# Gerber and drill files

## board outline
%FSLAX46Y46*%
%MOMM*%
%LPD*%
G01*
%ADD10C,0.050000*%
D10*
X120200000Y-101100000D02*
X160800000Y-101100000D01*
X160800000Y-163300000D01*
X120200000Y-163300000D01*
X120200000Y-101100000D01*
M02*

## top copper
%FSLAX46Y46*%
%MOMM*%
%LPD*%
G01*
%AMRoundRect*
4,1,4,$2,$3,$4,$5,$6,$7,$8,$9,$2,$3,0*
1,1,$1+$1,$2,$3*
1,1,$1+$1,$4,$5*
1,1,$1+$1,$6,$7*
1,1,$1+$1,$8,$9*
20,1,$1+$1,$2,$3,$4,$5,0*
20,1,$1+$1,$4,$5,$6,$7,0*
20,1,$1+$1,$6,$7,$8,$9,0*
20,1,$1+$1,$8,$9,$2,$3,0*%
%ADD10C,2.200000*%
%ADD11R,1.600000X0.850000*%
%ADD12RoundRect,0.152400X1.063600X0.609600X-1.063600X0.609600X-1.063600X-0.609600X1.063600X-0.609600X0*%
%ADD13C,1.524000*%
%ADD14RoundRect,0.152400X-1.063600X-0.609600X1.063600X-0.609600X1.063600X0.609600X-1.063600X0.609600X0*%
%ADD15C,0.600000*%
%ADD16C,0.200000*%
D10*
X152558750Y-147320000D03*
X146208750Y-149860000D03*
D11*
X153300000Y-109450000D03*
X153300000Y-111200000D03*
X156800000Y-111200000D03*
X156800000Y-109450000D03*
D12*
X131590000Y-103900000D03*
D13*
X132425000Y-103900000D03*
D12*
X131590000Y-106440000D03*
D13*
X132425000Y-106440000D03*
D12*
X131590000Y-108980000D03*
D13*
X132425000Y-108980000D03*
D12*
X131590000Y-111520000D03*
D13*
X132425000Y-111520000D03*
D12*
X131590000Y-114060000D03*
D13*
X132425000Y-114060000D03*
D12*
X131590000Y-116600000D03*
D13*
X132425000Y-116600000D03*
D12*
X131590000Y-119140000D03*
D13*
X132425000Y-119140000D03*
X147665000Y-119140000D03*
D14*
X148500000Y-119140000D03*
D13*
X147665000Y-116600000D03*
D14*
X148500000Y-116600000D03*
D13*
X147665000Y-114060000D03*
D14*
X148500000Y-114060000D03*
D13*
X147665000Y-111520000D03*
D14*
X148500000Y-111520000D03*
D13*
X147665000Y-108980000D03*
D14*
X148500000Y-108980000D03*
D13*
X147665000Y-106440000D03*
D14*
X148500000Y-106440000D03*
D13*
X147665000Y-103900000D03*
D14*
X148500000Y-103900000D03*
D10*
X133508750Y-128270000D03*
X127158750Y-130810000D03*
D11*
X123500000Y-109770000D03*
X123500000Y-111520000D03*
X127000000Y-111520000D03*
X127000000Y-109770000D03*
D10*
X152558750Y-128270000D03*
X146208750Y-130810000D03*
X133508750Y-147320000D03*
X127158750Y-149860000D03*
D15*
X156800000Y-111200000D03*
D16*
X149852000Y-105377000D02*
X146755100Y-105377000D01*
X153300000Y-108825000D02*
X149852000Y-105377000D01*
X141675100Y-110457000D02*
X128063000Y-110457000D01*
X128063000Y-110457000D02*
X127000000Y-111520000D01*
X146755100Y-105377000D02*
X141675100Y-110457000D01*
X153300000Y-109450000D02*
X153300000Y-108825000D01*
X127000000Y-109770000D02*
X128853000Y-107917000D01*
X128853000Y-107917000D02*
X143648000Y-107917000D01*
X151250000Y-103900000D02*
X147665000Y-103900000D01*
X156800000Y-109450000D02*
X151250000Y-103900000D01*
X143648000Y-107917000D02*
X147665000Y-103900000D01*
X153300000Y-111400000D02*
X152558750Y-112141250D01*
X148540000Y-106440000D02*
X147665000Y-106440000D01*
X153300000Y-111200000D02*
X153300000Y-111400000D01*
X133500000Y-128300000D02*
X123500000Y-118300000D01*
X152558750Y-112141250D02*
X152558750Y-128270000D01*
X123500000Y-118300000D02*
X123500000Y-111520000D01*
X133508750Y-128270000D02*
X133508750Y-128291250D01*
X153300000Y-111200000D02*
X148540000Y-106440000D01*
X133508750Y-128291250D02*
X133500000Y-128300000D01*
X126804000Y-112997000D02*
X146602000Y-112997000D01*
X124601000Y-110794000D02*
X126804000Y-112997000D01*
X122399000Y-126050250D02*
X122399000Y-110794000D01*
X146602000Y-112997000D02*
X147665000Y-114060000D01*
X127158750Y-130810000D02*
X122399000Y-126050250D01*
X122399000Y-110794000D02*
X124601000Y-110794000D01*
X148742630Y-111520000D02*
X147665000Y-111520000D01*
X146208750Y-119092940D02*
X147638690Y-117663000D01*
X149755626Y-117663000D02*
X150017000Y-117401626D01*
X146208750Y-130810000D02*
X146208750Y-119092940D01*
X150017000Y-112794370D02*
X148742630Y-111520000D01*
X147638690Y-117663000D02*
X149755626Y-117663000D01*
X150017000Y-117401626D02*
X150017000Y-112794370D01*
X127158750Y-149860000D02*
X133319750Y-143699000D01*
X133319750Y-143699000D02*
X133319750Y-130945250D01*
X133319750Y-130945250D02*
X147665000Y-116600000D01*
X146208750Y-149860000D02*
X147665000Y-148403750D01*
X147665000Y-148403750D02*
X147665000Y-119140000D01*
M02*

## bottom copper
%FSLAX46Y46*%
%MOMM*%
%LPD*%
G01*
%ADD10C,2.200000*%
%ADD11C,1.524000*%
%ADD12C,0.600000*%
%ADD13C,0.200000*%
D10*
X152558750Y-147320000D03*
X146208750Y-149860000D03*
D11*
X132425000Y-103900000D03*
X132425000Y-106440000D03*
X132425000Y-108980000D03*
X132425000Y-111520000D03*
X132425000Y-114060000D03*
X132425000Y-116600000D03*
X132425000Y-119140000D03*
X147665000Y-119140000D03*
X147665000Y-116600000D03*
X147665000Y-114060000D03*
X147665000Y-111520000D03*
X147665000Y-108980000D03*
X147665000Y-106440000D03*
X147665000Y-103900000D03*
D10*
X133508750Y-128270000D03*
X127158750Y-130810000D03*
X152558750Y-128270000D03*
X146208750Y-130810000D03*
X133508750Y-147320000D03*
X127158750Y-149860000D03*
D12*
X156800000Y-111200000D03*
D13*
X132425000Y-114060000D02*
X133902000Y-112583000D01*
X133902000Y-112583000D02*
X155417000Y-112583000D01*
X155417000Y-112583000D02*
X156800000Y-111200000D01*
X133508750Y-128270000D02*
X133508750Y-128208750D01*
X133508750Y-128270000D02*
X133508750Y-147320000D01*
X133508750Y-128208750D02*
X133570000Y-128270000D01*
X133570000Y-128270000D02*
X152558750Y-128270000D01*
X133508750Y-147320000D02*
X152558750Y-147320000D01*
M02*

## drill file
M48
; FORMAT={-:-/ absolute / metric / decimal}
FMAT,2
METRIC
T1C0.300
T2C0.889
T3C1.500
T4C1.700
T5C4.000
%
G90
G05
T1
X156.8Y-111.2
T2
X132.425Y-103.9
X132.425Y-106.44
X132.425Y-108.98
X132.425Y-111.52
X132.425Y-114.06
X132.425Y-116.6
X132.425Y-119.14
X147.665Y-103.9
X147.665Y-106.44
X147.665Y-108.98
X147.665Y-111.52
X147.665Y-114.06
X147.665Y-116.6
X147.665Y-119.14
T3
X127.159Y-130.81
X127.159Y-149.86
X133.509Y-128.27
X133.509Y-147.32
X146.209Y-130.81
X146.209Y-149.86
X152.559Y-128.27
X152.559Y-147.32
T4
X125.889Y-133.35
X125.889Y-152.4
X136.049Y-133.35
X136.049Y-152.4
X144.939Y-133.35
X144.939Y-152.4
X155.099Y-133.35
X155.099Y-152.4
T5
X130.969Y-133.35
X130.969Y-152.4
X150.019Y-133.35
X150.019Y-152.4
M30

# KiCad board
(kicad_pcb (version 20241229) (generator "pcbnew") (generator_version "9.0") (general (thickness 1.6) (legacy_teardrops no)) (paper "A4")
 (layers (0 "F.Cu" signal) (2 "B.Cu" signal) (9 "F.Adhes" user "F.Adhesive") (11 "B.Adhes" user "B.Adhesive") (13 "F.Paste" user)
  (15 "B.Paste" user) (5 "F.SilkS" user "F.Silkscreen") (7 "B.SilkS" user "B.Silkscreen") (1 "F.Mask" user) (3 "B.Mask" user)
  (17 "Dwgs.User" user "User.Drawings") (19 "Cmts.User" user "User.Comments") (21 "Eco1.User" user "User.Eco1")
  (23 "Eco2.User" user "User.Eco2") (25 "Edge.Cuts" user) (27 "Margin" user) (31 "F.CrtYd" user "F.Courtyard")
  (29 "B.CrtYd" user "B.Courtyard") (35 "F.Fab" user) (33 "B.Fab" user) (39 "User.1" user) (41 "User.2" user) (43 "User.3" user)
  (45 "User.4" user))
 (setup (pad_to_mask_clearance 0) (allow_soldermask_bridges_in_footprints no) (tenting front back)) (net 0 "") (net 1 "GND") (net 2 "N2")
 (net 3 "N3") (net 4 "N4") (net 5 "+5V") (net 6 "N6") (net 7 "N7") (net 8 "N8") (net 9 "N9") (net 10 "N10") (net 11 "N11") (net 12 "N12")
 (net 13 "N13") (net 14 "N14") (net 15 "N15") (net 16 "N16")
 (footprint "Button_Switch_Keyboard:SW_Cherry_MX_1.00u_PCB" (layer "F.Cu") (at 152.55875 147.32)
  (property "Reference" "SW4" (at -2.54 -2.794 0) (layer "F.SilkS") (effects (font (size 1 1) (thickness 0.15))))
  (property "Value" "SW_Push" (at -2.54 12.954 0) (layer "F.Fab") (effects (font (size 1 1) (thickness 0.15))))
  (pad "" np_thru_hole circle (at -7.62 5.08) (size 1.7 1.7) (drill 1.7) (layers "*.Cu" "*.Mask"))
  (pad "" np_thru_hole circle (at -2.54 5.08) (size 4 4) (drill 4) (layers "*.Cu" "*.Mask"))
  (pad "" np_thru_hole circle (at 2.54 5.08) (size 1.7 1.7) (drill 1.7) (layers "*.Cu" "*.Mask"))
  (pad "1" thru_hole circle (at 0 0) (size 2.2 2.2) (drill 1.5) (layers "*.Cu" "*.Mask") (remove_unused_layers no) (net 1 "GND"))
  (pad "2" thru_hole circle (at -6.35 2.54) (size 2.2 2.2) (drill 1.5) (layers "*.Cu" "*.Mask") (remove_unused_layers no) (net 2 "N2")))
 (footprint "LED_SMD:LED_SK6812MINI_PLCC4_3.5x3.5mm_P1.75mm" (layer "F.Cu") (at 155.05 110.325)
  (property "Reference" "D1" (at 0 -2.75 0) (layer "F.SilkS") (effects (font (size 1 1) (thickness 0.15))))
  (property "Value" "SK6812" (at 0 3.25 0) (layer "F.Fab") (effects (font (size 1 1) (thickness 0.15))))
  (pad "1" smd rect (at -1.75 -0.875) (size 1.6 0.85) (layers "F.Cu" "F.Mask" "F.Paste") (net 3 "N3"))
  (pad "2" smd rect (at -1.75 0.875) (size 1.6 0.85) (layers "F.Cu" "F.Mask" "F.Paste") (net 1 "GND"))
  (pad "3" smd rect (at 1.75 0.875) (size 1.6 0.85) (layers "F.Cu" "F.Mask" "F.Paste") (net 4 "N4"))
  (pad "4" smd rect (at 1.75 -0.875) (size 1.6 0.85) (layers "F.Cu" "F.Mask" "F.Paste") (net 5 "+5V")))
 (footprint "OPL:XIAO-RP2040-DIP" (layer "F.Cu") (at 140.045 111.52)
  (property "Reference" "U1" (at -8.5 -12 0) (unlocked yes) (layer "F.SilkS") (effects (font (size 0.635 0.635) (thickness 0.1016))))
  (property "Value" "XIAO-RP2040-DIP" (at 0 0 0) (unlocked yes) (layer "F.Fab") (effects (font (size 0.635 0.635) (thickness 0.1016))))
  (pad "1" smd roundrect (at -8.455 -7.62 180) (size 2.432 1.524) (layers "F.Cu" "F.Mask") (roundrect_rratio 0.1) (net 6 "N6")
   (thermal_bridge_angle 45))
  (pad "1" thru_hole circle (at -7.62 -7.62 180) (size 1.524 1.524) (drill 0.889) (layers "*.Cu" "*.Mask") (remove_unused_layers no)
   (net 6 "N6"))
  (pad "2" smd roundrect (at -8.455 -5.08 180) (size 2.432 1.524) (layers "F.Cu" "F.Mask") (roundrect_rratio 0.1) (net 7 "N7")
   (thermal_bridge_angle 45))
  (pad "2" thru_hole circle (at -7.62 -5.08 180) (size 1.524 1.524) (drill 0.889) (layers "*.Cu" "*.Mask") (remove_unused_layers no)
   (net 7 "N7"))
  (pad "3" smd roundrect (at -8.455 -2.54 180) (size 2.432 1.524) (layers "F.Cu" "F.Mask") (roundrect_rratio 0.1) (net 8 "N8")
   (thermal_bridge_angle 45))
  (pad "3" thru_hole circle (at -7.62 -2.54 180) (size 1.524 1.524) (drill 0.889) (layers "*.Cu" "*.Mask") (remove_unused_layers no)
   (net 8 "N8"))
  (pad "4" smd roundrect (at -8.455 0 180) (size 2.432 1.524) (layers "F.Cu" "F.Mask") (roundrect_rratio 0.1) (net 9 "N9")
   (thermal_bridge_angle 45))
  (pad "4" thru_hole circle (at -7.62 0 180) (size 1.524 1.524) (drill 0.889) (layers "*.Cu" "*.Mask") (remove_unused_layers no)
   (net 9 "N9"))
  (pad "5" smd roundrect (at -8.455 2.54 180) (size 2.432 1.524) (layers "F.Cu" "F.Mask") (roundrect_rratio 0.1) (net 4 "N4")
   (thermal_bridge_angle 45))
  (pad "5" thru_hole circle (at -7.62 2.54 180) (size 1.524 1.524) (drill 0.889) (layers "*.Cu" "*.Mask") (remove_unused_layers no)
   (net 4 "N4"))
  (pad "6" smd roundrect (at -8.455 5.08 180) (size 2.432 1.524) (layers "F.Cu" "F.Mask") (roundrect_rratio 0.1) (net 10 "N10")
   (thermal_bridge_angle 45))
  (pad "6" thru_hole circle (at -7.62 5.08 180) (size 1.524 1.524) (drill 0.889) (layers "*.Cu" "*.Mask") (remove_unused_layers no)
   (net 10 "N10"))
  (pad "7" smd roundrect (at -8.455 7.62 180) (size 2.432 1.524) (layers "F.Cu" "F.Mask") (roundrect_rratio 0.1) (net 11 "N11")
   (thermal_bridge_angle 45))
  (pad "7" thru_hole circle (at -7.62 7.62 180) (size 1.524 1.524) (drill 0.889) (layers "*.Cu" "*.Mask") (remove_unused_layers no)
   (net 11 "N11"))
  (pad "8" thru_hole circle (at 7.62 7.62) (size 1.524 1.524) (drill 0.889) (layers "*.Cu" "*.Mask") (remove_unused_layers no) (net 2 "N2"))
  (pad "8" smd roundrect (at 8.455 7.62) (size 2.432 1.524) (layers "F.Cu" "F.Mask") (roundrect_rratio 0.1) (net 2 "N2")
   (thermal_bridge_angle 45))
  (pad "9" thru_hole circle (at 7.62 5.08) (size 1.524 1.524) (drill 0.889) (layers "*.Cu" "*.Mask") (remove_unused_layers no)
   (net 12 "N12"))
  (pad "9" smd roundrect (at 8.455 5.08) (size 2.432 1.524) (layers "F.Cu" "F.Mask") (roundrect_rratio 0.1) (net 12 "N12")
   (thermal_bridge_angle 45))
  (pad "10" thru_hole circle (at 7.62 2.54) (size 1.524 1.524) (drill 0.889) (layers "*.Cu" "*.Mask") (remove_unused_layers no)
   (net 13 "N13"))
  (pad "10" smd roundrect (at 8.455 2.54) (size 2.432 1.524) (layers "F.Cu" "F.Mask") (roundrect_rratio 0.1) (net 13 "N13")
   (thermal_bridge_angle 45))
  (pad "11" thru_hole circle (at 7.62 0) (size 1.524 1.524) (drill 0.889) (layers "*.Cu" "*.Mask") (remove_unused_layers no) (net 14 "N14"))
  (pad "11" smd roundrect (at 8.455 0) (size 2.432 1.524) (layers "F.Cu" "F.Mask") (roundrect_rratio 0.1) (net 14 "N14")
   (thermal_bridge_angle 45))
  (pad "12" thru_hole circle (at 7.62 -2.54) (size 1.524 1.524) (drill 0.889) (layers "*.Cu" "*.Mask") (remove_unused_layers no)
   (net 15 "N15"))
  (pad "12" smd roundrect (at 8.455 -2.54) (size 2.432 1.524) (layers "F.Cu" "F.Mask") (roundrect_rratio 0.1) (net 15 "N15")
   (thermal_bridge_angle 45))
  (pad "13" thru_hole circle (at 7.62 -5.08) (size 1.524 1.524) (drill 0.889) (layers "*.Cu" "*.Mask") (remove_unused_layers no)
   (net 1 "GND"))
  (pad "13" smd roundrect (at 8.455 -5.08) (size 2.432 1.524) (layers "F.Cu" "F.Mask") (roundrect_rratio 0.1) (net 1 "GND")
   (thermal_bridge_angle 45))
  (pad "14" thru_hole circle (at 7.62 -7.62) (size 1.524 1.524) (drill 0.889) (layers "*.Cu" "*.Mask") (remove_unused_layers no)
   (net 5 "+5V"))
  (pad "14" smd roundrect (at 8.455 -7.62) (size 2.432 1.524) (layers "F.Cu" "F.Mask") (roundrect_rratio 0.1) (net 5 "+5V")
   (thermal_bridge_angle 45)))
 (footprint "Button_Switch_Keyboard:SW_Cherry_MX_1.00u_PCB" (layer "F.Cu") (at 133.50875 128.27)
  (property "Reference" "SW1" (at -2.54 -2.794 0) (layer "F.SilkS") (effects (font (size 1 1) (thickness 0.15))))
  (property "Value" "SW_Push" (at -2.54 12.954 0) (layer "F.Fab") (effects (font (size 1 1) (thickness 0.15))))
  (pad "" np_thru_hole circle (at -7.62 5.08) (size 1.7 1.7) (drill 1.7) (layers "*.Cu" "*.Mask"))
  (pad "" np_thru_hole circle (at -2.54 5.08) (size 4 4) (drill 4) (layers "*.Cu" "*.Mask"))
  (pad "" np_thru_hole circle (at 2.54 5.08) (size 1.7 1.7) (drill 1.7) (layers "*.Cu" "*.Mask"))
  (pad "1" thru_hole circle (at 0 0) (size 2.2 2.2) (drill 1.5) (layers "*.Cu" "*.Mask") (remove_unused_layers no) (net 1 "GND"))
  (pad "2" thru_hole circle (at -6.35 2.54) (size 2.2 2.2) (drill 1.5) (layers "*.Cu" "*.Mask") (remove_unused_layers no) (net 13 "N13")))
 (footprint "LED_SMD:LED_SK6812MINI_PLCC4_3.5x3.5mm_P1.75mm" (layer "F.Cu") (at 125.25 110.645)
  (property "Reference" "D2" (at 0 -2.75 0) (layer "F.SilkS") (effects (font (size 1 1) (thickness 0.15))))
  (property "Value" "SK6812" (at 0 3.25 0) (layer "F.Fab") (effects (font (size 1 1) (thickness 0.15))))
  (pad "1" smd rect (at -1.75 -0.875) (size 1.6 0.85) (layers "F.Cu" "F.Mask" "F.Paste") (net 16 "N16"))
  (pad "2" smd rect (at -1.75 0.875) (size 1.6 0.85) (layers "F.Cu" "F.Mask" "F.Paste") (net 1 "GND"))
  (pad "3" smd rect (at 1.75 0.875) (size 1.6 0.85) (layers "F.Cu" "F.Mask" "F.Paste") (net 3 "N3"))
  (pad "4" smd rect (at 1.75 -0.875) (size 1.6 0.85) (layers "F.Cu" "F.Mask" "F.Paste") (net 5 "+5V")))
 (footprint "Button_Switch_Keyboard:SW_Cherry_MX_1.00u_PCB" (layer "F.Cu") (at 152.55875 128.27)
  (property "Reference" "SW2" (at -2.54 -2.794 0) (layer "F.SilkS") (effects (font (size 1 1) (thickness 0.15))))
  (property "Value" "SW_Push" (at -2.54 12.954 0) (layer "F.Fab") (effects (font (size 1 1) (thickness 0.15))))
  (pad "" np_thru_hole circle (at -7.62 5.08) (size 1.7 1.7) (drill 1.7) (layers "*.Cu" "*.Mask"))
  (pad "" np_thru_hole circle (at -2.54 5.08) (size 4 4) (drill 4) (layers "*.Cu" "*.Mask"))
  (pad "" np_thru_hole circle (at 2.54 5.08) (size 1.7 1.7) (drill 1.7) (layers "*.Cu" "*.Mask"))
  (pad "1" thru_hole circle (at 0 0) (size 2.2 2.2) (drill 1.5) (layers "*.Cu" "*.Mask") (remove_unused_layers no) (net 1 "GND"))
  (pad "2" thru_hole circle (at -6.35 2.54) (size 2.2 2.2) (drill 1.5) (layers "*.Cu" "*.Mask") (remove_unused_layers no) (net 14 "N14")))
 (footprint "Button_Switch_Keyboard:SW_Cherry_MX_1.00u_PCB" (layer "F.Cu") (at 133.50875 147.32)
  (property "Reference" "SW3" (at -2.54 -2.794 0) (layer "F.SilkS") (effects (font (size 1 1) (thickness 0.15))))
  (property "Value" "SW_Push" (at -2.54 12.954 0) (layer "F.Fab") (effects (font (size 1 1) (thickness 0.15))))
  (pad "" np_thru_hole circle (at -7.62 5.08) (size 1.7 1.7) (drill 1.7) (layers "*.Cu" "*.Mask"))
  (pad "" np_thru_hole circle (at -2.54 5.08) (size 4 4) (drill 4) (layers "*.Cu" "*.Mask"))
  (pad "" np_thru_hole circle (at 2.54 5.08) (size 1.7 1.7) (drill 1.7) (layers "*.Cu" "*.Mask"))
  (pad "1" thru_hole circle (at 0 0) (size 2.2 2.2) (drill 1.5) (layers "*.Cu" "*.Mask") (remove_unused_layers no) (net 1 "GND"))
  (pad "2" thru_hole circle (at -6.35 2.54) (size 2.2 2.2) (drill 1.5) (layers "*.Cu" "*.Mask") (remove_unused_layers no) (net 12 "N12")))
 (gr_rect (start 120.2 101.1) (end 160.8 163.3) (stroke (width 0.05) (type default)) (fill no) (layer "Edge.Cuts"))
 (segment (start 149.852 105.377) (end 146.7551 105.377) (width 0.2) (layer "F.Cu") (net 3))
 (segment (start 153.3 108.825) (end 149.852 105.377) (width 0.2) (layer "F.Cu") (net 3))
 (segment (start 141.6751 110.457) (end 128.063 110.457) (width 0.2) (layer "F.Cu") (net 3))
 (segment (start 128.063 110.457) (end 127 111.52) (width 0.2) (layer "F.Cu") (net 3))
 (segment (start 146.7551 105.377) (end 141.6751 110.457) (width 0.2) (layer "F.Cu") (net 3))
 (segment (start 153.3 109.45) (end 153.3 108.825) (width 0.2) (layer "F.Cu") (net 3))
 (via (at 156.8 111.2) (size 0.6) (drill 0.3) (layers "F.Cu" "B.Cu") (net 4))
 (segment (start 132.425 114.06) (end 133.902 112.583) (width 0.2) (layer "B.Cu") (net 4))
 (segment (start 133.902 112.583) (end 155.417 112.583) (width 0.2) (layer "B.Cu") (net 4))
 (segment (start 155.417 112.583) (end 156.8 111.2) (width 0.2) (layer "B.Cu") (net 4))
 (segment (start 127 109.77) (end 128.853 107.917) (width 0.2) (layer "F.Cu") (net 5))
 (segment (start 128.853 107.917) (end 143.648 107.917) (width 0.2) (layer "F.Cu") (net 5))
 (segment (start 151.25 103.9) (end 147.665 103.9) (width 0.2) (layer "F.Cu") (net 5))
 (segment (start 156.8 109.45) (end 151.25 103.9) (width 0.2) (layer "F.Cu") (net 5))
 (segment (start 143.648 107.917) (end 147.665 103.9) (width 0.2) (layer "F.Cu") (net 5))
 (segment (start 153.3 111.4) (end 152.55875 112.14125) (width 0.2) (layer "F.Cu") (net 1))
 (segment (start 148.54 106.44) (end 147.665 106.44) (width 0.2) (layer "F.Cu") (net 1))
 (segment (start 153.3 111.2) (end 153.3 111.4) (width 0.2) (layer "F.Cu") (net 1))
 (segment (start 133.5 128.3) (end 123.5 118.3) (width 0.2) (layer "F.Cu") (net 1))
 (segment (start 152.55875 112.14125) (end 152.55875 128.27) (width 0.2) (layer "F.Cu") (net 1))
 (segment (start 123.5 118.3) (end 123.5 111.52) (width 0.2) (layer "F.Cu") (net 1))
 (segment (start 133.50875 128.27) (end 133.50875 128.29125) (width 0.2) (layer "F.Cu") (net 1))
 (segment (start 153.3 111.2) (end 148.54 106.44) (width 0.2) (layer "F.Cu") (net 1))
 (segment (start 133.50875 128.29125) (end 133.5 128.3) (width 0.2) (layer "F.Cu") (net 1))
 (segment (start 133.50875 128.27) (end 133.50875 128.20875) (width 0.2) (layer "B.Cu") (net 1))
 (segment (start 133.50875 128.27) (end 133.50875 147.32) (width 0.2) (layer "B.Cu") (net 1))
 (segment (start 133.50875 128.20875) (end 133.57 128.27) (width 0.2) (layer "B.Cu") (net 1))
 (segment (start 133.57 128.27) (end 152.55875 128.27) (width 0.2) (layer "B.Cu") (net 1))
 (segment (start 133.50875 147.32) (end 152.55875 147.32) (width 0.2) (layer "B.Cu") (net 1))
 (segment (start 126.804 112.997) (end 146.602 112.997) (width 0.2) (layer "F.Cu") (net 13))
 (segment (start 124.601 110.794) (end 126.804 112.997) (width 0.2) (layer "F.Cu") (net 13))
 (segment (start 122.399 126.05025) (end 122.399 110.794) (width 0.2) (layer "F.Cu") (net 13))
 (segment (start 146.602 112.997) (end 147.665 114.06) (width 0.2) (layer "F.Cu") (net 13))
 (segment (start 127.15875 130.81) (end 122.399 126.05025) (width 0.2) (layer "F.Cu") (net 13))
 (segment (start 122.399 110.794) (end 124.601 110.794) (width 0.2) (layer "F.Cu") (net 13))
 (segment (start 148.74263 111.52) (end 147.665 111.52) (width 0.2) (layer "F.Cu") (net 14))
 (segment (start 146.20875 119.09294) (end 147.63869 117.663) (width 0.2) (layer "F.Cu") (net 14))
 (segment (start 149.755626 117.663) (end 150.017 117.401626) (width 0.2) (layer "F.Cu") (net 14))
 (segment (start 146.20875 130.81) (end 146.20875 119.09294) (width 0.2) (layer "F.Cu") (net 14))
 (segment (start 150.017 112.79437) (end 148.74263 111.52) (width 0.2) (layer "F.Cu") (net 14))
 (segment (start 147.63869 117.663) (end 149.755626 117.663) (width 0.2) (layer "F.Cu") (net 14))
 (segment (start 150.017 117.401626) (end 150.017 112.79437) (width 0.2) (layer "F.Cu") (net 14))
 (segment (start 127.15875 149.86) (end 133.31975 143.699) (width 0.2) (layer "F.Cu") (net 12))
 (segment (start 133.31975 143.699) (end 133.31975 130.94525) (width 0.2) (layer "F.Cu") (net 12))
 (segment (start 133.31975 130.94525) (end 147.665 116.6) (width 0.2) (layer "F.Cu") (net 12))
 (segment (start 146.20875 149.86) (end 147.665 148.40375) (width 0.2) (layer "F.Cu") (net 2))
 (segment (start 147.665 148.40375) (end 147.665 119.14) (width 0.2) (layer "F.Cu") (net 2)))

